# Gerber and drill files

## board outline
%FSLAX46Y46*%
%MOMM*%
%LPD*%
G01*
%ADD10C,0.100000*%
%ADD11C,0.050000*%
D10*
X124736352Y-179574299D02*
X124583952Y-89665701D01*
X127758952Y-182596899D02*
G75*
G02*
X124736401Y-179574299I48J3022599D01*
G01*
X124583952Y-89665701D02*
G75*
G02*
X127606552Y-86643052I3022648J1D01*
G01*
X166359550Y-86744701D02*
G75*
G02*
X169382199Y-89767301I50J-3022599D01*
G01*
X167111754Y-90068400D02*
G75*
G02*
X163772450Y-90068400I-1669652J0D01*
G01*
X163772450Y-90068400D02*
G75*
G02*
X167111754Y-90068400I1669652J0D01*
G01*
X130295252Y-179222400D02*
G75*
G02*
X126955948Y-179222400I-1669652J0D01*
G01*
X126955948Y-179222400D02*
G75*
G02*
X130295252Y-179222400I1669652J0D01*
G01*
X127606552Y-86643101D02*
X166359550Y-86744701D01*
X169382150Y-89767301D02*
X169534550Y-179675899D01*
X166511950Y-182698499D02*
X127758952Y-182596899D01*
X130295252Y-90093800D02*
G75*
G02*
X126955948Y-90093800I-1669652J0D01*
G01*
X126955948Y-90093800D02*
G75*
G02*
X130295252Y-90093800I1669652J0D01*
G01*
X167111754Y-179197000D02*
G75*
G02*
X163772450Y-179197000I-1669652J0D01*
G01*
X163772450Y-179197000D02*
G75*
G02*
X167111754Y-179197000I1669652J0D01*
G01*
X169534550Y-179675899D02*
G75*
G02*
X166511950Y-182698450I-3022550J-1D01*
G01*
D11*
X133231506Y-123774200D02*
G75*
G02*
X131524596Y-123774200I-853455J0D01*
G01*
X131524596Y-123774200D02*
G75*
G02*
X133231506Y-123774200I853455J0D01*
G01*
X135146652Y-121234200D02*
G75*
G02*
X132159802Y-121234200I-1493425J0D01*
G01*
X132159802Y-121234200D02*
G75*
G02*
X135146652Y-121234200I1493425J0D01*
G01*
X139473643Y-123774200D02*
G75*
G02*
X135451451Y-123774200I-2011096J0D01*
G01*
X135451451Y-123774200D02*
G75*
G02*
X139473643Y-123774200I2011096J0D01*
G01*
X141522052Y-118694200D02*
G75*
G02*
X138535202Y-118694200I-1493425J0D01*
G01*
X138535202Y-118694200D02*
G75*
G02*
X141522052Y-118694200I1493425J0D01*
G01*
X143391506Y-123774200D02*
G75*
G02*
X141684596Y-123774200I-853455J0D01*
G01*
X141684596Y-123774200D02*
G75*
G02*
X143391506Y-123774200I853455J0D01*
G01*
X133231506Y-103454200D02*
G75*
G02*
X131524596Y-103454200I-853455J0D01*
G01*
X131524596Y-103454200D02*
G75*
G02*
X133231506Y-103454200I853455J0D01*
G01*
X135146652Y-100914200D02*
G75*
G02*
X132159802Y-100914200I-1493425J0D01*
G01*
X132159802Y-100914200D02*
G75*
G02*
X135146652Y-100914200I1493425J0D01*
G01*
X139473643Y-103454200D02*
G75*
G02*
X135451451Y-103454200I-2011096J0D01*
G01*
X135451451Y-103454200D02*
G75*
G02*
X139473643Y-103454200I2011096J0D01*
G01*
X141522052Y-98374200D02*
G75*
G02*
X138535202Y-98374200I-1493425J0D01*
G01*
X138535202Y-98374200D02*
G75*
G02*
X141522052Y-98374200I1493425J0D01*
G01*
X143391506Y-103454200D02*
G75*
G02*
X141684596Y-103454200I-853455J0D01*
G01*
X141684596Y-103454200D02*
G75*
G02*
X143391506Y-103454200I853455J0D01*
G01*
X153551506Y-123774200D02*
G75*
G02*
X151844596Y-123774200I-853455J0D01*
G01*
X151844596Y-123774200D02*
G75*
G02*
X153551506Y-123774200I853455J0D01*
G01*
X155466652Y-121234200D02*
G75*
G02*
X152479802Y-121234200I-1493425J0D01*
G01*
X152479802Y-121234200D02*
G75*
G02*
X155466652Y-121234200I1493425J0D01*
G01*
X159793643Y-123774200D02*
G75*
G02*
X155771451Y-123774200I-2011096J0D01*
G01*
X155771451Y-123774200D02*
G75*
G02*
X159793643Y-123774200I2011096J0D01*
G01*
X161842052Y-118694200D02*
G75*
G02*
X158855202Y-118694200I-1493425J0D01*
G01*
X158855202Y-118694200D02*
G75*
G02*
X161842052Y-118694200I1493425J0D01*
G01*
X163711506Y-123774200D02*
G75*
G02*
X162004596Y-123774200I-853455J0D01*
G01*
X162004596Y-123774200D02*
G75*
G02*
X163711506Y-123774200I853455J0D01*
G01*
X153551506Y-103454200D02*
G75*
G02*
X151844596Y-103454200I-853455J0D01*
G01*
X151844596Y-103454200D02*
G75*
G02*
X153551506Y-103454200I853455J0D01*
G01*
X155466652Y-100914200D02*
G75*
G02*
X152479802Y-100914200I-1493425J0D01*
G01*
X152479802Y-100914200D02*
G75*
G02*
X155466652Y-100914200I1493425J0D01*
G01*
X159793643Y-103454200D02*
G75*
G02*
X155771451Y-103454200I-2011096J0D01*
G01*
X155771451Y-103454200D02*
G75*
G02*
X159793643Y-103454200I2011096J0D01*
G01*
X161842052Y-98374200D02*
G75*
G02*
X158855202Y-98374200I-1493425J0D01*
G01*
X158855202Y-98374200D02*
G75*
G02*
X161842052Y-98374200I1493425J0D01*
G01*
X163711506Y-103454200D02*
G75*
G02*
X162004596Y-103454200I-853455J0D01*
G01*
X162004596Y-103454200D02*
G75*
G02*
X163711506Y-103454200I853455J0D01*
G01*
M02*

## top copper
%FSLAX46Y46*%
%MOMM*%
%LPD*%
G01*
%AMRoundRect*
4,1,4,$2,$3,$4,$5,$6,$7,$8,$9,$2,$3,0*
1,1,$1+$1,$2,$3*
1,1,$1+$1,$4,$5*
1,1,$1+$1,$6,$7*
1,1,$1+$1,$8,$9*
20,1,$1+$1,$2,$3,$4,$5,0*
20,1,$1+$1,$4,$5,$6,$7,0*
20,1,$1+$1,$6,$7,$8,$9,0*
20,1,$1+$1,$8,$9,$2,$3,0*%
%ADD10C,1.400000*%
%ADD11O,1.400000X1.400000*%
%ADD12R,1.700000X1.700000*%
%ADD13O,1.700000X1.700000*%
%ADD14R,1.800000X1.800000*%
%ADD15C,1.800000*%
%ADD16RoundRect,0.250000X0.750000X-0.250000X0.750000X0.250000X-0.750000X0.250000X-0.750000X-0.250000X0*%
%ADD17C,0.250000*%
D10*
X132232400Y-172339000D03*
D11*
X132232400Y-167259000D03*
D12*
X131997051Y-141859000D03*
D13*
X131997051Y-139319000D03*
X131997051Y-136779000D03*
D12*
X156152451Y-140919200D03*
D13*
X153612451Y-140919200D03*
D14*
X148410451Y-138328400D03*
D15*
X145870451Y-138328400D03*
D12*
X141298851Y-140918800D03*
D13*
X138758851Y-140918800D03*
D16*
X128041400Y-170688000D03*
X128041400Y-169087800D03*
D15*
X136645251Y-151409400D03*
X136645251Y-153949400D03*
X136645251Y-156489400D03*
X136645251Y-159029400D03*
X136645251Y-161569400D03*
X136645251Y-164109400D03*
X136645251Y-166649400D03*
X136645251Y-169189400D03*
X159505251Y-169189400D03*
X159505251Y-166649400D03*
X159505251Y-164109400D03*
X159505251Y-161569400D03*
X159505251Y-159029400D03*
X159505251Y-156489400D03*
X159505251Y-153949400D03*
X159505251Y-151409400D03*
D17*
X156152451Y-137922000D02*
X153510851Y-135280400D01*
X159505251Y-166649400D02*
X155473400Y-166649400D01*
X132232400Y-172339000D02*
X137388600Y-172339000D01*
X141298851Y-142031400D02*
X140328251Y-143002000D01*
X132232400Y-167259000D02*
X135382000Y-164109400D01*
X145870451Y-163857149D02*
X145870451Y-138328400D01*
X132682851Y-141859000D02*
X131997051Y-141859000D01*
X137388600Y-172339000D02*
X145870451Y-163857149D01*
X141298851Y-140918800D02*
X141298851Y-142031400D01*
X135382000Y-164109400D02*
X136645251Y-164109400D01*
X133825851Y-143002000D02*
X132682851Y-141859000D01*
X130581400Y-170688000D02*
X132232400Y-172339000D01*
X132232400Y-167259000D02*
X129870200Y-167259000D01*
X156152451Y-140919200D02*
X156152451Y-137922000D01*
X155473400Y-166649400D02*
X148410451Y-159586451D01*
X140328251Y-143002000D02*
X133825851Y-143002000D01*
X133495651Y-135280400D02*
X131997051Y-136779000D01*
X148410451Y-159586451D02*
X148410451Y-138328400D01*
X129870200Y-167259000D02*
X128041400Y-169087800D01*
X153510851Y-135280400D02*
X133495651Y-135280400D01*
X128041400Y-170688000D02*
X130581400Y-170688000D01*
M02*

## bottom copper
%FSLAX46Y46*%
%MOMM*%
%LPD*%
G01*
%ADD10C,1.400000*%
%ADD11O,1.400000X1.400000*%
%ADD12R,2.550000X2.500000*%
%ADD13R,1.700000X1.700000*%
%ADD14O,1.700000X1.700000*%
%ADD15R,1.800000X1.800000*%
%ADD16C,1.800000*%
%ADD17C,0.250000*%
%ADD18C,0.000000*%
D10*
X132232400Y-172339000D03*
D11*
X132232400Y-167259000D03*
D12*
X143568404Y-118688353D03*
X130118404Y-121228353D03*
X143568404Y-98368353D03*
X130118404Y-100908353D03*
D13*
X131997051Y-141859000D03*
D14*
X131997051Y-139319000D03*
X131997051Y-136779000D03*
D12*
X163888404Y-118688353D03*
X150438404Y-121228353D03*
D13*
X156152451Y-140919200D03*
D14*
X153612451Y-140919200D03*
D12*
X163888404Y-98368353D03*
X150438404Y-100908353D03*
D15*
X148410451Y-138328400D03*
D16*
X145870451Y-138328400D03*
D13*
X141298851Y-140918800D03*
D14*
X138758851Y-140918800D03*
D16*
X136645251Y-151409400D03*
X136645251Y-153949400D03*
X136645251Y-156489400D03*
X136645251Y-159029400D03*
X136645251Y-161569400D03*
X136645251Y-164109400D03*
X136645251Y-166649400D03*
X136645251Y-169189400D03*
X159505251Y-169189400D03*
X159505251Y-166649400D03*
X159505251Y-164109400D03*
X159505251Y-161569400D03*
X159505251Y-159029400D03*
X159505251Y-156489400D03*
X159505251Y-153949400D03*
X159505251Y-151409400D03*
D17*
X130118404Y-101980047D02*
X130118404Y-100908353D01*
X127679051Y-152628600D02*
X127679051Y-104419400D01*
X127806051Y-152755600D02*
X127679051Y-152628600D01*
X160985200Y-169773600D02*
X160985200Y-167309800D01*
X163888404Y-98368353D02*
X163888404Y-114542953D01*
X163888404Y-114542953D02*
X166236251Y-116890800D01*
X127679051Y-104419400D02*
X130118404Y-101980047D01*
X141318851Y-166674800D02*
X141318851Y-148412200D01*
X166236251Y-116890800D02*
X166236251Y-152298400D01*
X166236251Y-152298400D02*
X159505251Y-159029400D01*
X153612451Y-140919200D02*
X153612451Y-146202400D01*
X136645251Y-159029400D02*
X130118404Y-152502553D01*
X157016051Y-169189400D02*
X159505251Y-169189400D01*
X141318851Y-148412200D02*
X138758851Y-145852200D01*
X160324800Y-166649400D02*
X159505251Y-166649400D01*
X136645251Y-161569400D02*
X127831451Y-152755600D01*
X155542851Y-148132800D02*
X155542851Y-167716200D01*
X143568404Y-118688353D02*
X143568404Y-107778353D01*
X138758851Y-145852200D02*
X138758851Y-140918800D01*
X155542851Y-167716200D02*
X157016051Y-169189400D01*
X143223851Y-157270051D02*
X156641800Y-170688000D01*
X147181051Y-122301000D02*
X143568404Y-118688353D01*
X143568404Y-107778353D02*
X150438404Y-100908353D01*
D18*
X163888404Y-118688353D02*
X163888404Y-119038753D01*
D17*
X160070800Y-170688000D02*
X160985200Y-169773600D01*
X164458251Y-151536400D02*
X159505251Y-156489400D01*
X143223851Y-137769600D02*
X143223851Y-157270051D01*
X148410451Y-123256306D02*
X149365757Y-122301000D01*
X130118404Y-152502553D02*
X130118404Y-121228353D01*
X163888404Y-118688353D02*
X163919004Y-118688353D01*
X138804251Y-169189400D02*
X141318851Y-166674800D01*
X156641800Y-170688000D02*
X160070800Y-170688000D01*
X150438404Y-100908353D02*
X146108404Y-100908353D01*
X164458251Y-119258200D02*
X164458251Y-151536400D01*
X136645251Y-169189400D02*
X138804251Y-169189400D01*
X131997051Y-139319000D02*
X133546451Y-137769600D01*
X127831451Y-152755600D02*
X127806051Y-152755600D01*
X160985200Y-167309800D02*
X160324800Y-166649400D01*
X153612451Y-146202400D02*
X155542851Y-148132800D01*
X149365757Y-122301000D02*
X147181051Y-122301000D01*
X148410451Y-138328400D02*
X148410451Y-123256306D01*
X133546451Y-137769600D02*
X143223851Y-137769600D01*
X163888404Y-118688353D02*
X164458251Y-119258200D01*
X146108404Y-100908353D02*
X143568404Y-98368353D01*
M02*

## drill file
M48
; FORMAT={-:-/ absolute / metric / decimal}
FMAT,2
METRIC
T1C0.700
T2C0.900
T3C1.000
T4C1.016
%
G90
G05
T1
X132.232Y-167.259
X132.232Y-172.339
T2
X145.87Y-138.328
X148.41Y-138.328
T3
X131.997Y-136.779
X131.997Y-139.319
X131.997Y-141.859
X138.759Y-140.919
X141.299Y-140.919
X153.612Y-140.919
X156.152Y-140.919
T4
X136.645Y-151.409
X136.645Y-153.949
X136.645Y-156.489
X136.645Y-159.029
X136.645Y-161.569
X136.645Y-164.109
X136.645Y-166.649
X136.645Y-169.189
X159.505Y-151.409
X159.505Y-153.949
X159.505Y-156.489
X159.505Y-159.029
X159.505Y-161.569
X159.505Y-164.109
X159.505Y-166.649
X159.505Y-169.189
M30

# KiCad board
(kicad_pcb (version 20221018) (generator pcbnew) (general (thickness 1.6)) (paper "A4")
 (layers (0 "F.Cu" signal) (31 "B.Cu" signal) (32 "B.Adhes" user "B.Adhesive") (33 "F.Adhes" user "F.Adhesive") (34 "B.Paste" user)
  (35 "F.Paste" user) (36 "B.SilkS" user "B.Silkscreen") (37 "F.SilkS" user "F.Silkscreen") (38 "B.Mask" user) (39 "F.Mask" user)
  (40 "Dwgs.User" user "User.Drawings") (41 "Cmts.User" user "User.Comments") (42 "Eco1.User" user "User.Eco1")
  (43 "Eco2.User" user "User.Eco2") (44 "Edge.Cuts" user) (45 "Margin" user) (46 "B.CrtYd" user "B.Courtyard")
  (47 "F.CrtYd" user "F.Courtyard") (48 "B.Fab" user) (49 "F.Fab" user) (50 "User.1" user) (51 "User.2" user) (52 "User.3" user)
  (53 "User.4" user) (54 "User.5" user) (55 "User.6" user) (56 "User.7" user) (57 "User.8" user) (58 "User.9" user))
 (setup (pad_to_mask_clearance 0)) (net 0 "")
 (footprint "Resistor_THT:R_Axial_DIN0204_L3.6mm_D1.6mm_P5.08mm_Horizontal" (layer "F.Cu") (at 132.2324 172.339 90)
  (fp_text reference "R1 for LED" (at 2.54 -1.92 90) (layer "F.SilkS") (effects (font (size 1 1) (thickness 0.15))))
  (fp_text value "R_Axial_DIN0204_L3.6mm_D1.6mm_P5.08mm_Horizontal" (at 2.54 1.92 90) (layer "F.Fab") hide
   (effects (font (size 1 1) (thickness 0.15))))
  (pad "1" thru_hole circle (at 0 0 90) (size 1.4 1.4) (drill 0.7) (layers "*.Cu" "*.Mask"))
  (pad "2" thru_hole oval (at 5.08 0 90) (size 1.4 1.4) (drill 0.7) (layers "*.Cu" "*.Mask")))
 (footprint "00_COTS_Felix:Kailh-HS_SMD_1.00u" (layer "F.Cu") (at 137.458051 123.7742)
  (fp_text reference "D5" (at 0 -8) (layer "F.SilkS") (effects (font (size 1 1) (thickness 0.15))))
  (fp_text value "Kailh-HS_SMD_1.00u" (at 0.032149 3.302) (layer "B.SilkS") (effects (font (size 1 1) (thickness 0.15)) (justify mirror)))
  (fp_circle (center -5.08 0) (end -4.572 -0.6858) (stroke (width 0.05) (type default)) (fill none) (layer "Edge.Cuts"))
  (fp_circle (center -3.804824 -2.54) (end -2.687224 -3.5306) (stroke (width 0.05) (type default)) (fill none) (layer "Edge.Cuts"))
  (fp_circle (center 0.004496 0) (end 0.944296 -1.778) (stroke (width 0.05) (type default)) (fill none) (layer "Edge.Cuts"))
  (fp_circle (center 2.570576 -5.08) (end 4.064001 -5.08) (stroke (width 0.05) (type default)) (fill none) (layer "Edge.Cuts"))
  (fp_circle (center 5.08 0) (end 5.588 -0.6858) (stroke (width 0.05) (type default)) (fill none) (layer "Edge.Cuts"))
  (pad "1" smd rect (at 6.110353 -5.085847) (size 2.55 2.5) (layers "B.Cu" "F.Paste" "F.Mask") (solder_mask_margin 0.102))
  (pad "2" smd rect (at -7.339647 -2.545847) (size 2.55 2.5) (layers "B.Cu" "F.Paste" "F.Mask") (solder_mask_margin 0.102)))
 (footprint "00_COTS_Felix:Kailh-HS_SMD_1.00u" (layer "F.Cu") (at 137.458051 103.4542)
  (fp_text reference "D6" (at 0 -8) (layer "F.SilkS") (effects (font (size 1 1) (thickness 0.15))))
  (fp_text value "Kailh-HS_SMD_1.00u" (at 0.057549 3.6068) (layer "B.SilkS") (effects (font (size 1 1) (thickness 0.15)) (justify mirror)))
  (fp_circle (center -5.08 0) (end -4.572 -0.6858) (stroke (width 0.05) (type default)) (fill none) (layer "Edge.Cuts"))
  (fp_circle (center -3.804824 -2.54) (end -2.687224 -3.5306) (stroke (width 0.05) (type default)) (fill none) (layer "Edge.Cuts"))
  (fp_circle (center 0.004496 0) (end 0.944296 -1.778) (stroke (width 0.05) (type default)) (fill none) (layer "Edge.Cuts"))
  (fp_circle (center 2.570576 -5.08) (end 4.064001 -5.08) (stroke (width 0.05) (type default)) (fill none) (layer "Edge.Cuts"))
  (fp_circle (center 5.08 0) (end 5.588 -0.6858) (stroke (width 0.05) (type default)) (fill none) (layer "Edge.Cuts"))
  (pad "1" smd rect (at 6.110353 -5.085847) (size 2.55 2.5) (layers "B.Cu" "F.Paste" "F.Mask") (solder_mask_margin 0.102))
  (pad "2" smd rect (at -7.339647 -2.545847) (size 2.55 2.5) (layers "B.Cu" "F.Paste" "F.Mask") (solder_mask_margin 0.102)))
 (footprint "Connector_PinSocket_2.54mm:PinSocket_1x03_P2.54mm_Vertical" (layer "F.Cu") (at 131.997051 141.859 180)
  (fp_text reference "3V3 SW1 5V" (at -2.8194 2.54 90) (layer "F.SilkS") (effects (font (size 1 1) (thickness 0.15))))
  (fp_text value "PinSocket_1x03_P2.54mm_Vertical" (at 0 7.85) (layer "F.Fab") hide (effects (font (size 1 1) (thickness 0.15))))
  (pad "1" thru_hole rect (at 0 0 180) (size 1.7 1.7) (drill 1) (layers "*.Cu" "*.Mask"))
  (pad "2" thru_hole oval (at 0 2.54 180) (size 1.7 1.7) (drill 1) (layers "*.Cu" "*.Mask"))
  (pad "3" thru_hole oval (at 0 5.08 180) (size 1.7 1.7) (drill 1) (layers "*.Cu" "*.Mask")))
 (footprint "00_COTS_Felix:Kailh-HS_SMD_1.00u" (layer "F.Cu") (at 157.778051 123.7742)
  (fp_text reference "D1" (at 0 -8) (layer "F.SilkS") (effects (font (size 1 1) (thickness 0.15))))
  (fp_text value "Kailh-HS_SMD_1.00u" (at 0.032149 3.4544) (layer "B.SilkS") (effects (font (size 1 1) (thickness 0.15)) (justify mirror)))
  (fp_circle (center -5.08 0) (end -4.572 -0.6858) (stroke (width 0.05) (type default)) (fill none) (layer "Edge.Cuts"))
  (fp_circle (center -3.804824 -2.54) (end -2.687224 -3.5306) (stroke (width 0.05) (type default)) (fill none) (layer "Edge.Cuts"))
  (fp_circle (center 0.004496 0) (end 0.944296 -1.778) (stroke (width 0.05) (type default)) (fill none) (layer "Edge.Cuts"))
  (fp_circle (center 2.570576 -5.08) (end 4.064001 -5.08) (stroke (width 0.05) (type default)) (fill none) (layer "Edge.Cuts"))
  (fp_circle (center 5.08 0) (end 5.588 -0.6858) (stroke (width 0.05) (type default)) (fill none) (layer "Edge.Cuts"))
  (pad "1" smd rect (at 6.110353 -5.085847) (size 2.55 2.5) (layers "B.Cu" "F.Paste" "F.Mask") (solder_mask_margin 0.102))
  (pad "2" smd rect (at -7.339647 -2.545847) (size 2.55 2.5) (layers "B.Cu" "F.Paste" "F.Mask") (solder_mask_margin 0.102)))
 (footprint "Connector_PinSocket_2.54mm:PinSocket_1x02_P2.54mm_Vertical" (layer "F.Cu") (at 156.152451 140.9192 -90)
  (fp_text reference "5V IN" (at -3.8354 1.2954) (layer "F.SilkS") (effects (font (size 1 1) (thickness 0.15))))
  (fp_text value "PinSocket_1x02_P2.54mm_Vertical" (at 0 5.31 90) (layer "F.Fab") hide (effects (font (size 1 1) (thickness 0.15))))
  (pad "1" thru_hole rect (at 0 0 270) (size 1.7 1.7) (drill 1) (layers "*.Cu" "*.Mask"))
  (pad "2" thru_hole oval (at 0 2.54 270) (size 1.7 1.7) (drill 1) (layers "*.Cu" "*.Mask")))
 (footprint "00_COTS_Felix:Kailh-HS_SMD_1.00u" (layer "F.Cu") (at 157.778051 103.4542)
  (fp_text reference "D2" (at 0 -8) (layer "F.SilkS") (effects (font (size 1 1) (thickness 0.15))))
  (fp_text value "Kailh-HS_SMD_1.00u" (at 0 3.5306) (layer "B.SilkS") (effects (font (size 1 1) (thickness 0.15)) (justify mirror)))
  (fp_circle (center -5.08 0) (end -4.572 -0.6858) (stroke (width 0.05) (type default)) (fill none) (layer "Edge.Cuts"))
  (fp_circle (center -3.804824 -2.54) (end -2.687224 -3.5306) (stroke (width 0.05) (type default)) (fill none) (layer "Edge.Cuts"))
  (fp_circle (center 0.004496 0) (end 0.944296 -1.778) (stroke (width 0.05) (type default)) (fill none) (layer "Edge.Cuts"))
  (fp_circle (center 2.570576 -5.08) (end 4.064001 -5.08) (stroke (width 0.05) (type default)) (fill none) (layer "Edge.Cuts"))
  (fp_circle (center 5.08 0) (end 5.588 -0.6858) (stroke (width 0.05) (type default)) (fill none) (layer "Edge.Cuts"))
  (pad "1" smd rect (at 6.110353 -5.085847) (size 2.55 2.5) (layers "B.Cu" "F.Paste" "F.Mask") (solder_mask_margin 0.102))
  (pad "2" smd rect (at -7.339647 -2.545847) (size 2.55 2.5) (layers "B.Cu" "F.Paste" "F.Mask") (solder_mask_margin 0.102)))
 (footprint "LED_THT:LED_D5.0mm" (layer "F.Cu") (at 148.410451 138.3284 180)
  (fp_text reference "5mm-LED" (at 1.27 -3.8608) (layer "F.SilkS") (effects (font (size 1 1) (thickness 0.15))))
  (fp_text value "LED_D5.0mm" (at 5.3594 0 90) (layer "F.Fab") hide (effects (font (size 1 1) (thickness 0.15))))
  (pad "1" thru_hole rect (at 0 0 180) (size 1.8 1.8) (drill 0.9) (layers "*.Cu" "*.Mask"))
  (pad "2" thru_hole circle (at 2.54 0 180) (size 1.8 1.8) (drill 0.9) (layers "*.Cu" "*.Mask")))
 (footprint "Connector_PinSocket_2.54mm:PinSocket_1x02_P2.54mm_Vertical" (layer "F.Cu") (at 141.298851 140.9188 -90)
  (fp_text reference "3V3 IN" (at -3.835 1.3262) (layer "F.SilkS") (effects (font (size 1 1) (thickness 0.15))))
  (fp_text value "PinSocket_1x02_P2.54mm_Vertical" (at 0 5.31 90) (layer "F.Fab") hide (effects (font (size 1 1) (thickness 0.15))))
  (pad "1" thru_hole rect (at 0 0 270) (size 1.7 1.7) (drill 1) (layers "*.Cu" "*.Mask"))
  (pad "2" thru_hole oval (at 0 2.54 270) (size 1.7 1.7) (drill 1) (layers "*.Cu" "*.Mask")))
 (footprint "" (layer "F.Cu") (at 128.0414 170.688)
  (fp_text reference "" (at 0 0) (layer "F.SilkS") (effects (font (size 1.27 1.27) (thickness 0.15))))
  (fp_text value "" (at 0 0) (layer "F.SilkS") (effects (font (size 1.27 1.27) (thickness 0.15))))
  (pad "1" smd roundrect (at 0 0 90) (size 1 2) (layers "F.Cu" "F.Paste" "F.Mask") (roundrect_rratio 0.25)))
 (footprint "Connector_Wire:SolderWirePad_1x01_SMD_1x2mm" (layer "F.Cu") (at 128.0414 169.0878 90)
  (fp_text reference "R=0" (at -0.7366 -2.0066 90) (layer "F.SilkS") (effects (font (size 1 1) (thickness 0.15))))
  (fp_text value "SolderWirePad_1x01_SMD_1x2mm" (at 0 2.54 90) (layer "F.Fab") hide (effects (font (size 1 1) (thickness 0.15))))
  (pad "1" smd roundrect (at 0 0 90) (size 1 2) (layers "F.Cu" "F.Paste" "F.Mask") (roundrect_rratio 0.25)))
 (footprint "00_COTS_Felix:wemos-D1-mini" (layer "F.Cu") (at 148.088051 160.6542)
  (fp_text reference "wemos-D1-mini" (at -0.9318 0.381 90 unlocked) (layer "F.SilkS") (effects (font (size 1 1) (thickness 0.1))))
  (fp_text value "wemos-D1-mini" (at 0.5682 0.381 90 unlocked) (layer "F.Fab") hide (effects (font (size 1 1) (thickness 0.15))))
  (pad "1" thru_hole circle (at -11.4428 -9.2448 90) (size 1.8 1.8) (drill 1.016) (layers "*.Cu" "*.Mask"))
  (pad "2" thru_hole circle (at -11.4428 -6.7048 90) (size 1.8 1.8) (drill 1.016) (layers "*.Cu" "*.Mask"))
  (pad "3" thru_hole circle (at -11.4428 -4.1648 90) (size 1.8 1.8) (drill 1.016) (layers "*.Cu" "*.Mask"))
  (pad "4" thru_hole circle (at -11.4428 -1.6248 90) (size 1.8 1.8) (drill 1.016) (layers "*.Cu" "*.Mask"))
  (pad "5" thru_hole circle (at -11.4428 0.9152 90) (size 1.8 1.8) (drill 1.016) (layers "*.Cu" "*.Mask"))
  (pad "6" thru_hole circle (at -11.4428 3.4552 90) (size 1.8 1.8) (drill 1.016) (layers "*.Cu" "*.Mask"))
  (pad "7" thru_hole circle (at -11.4428 5.9952 90) (size 1.8 1.8) (drill 1.016) (layers "*.Cu" "*.Mask"))
  (pad "8" thru_hole circle (at -11.4428 8.5352 90) (size 1.8 1.8) (drill 1.016) (layers "*.Cu" "*.Mask"))
  (pad "9" thru_hole circle (at 11.4172 8.5352 90) (size 1.8 1.8) (drill 1.016) (layers "*.Cu" "*.Mask"))
  (pad "10" thru_hole circle (at 11.4172 5.9952 90) (size 1.8 1.8) (drill 1.016) (layers "*.Cu" "*.Mask"))
  (pad "11" thru_hole circle (at 11.4172 3.4552 90) (size 1.8 1.8) (drill 1.016) (layers "*.Cu" "*.Mask"))
  (pad "12" thru_hole circle (at 11.4172 0.9152 90) (size 1.8 1.8) (drill 1.016) (layers "*.Cu" "*.Mask"))
  (pad "13" thru_hole circle (at 11.4172 -1.6248 90) (size 1.8 1.8) (drill 1.016) (layers "*.Cu" "*.Mask"))
  (pad "14" thru_hole circle (at 11.4172 -4.1648 90) (size 1.8 1.8) (drill 1.016) (layers "*.Cu" "*.Mask"))
  (pad "15" thru_hole circle (at 11.4172 -6.7048 90) (size 1.8 1.8) (drill 1.016) (layers "*.Cu" "*.Mask"))
  (pad "16" thru_hole circle (at 11.4172 -9.2448 90) (size 1.8 1.8) (drill 1.016) (layers "*.Cu" "*.Mask")))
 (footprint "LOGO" (layer "B.Cu") (at 147.2184 114.0206 180)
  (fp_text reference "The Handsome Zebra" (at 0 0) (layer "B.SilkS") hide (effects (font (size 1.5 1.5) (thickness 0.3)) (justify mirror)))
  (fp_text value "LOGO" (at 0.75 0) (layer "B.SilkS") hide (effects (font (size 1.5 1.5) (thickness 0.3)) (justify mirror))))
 (gr_line (start 124.736352 179.574299) (end 124.583952 89.665701) (stroke (width 0.1) (type default)) (layer "Edge.Cuts"))
 (gr_arc (start 127.758952 182.596899) (mid 125.621651 181.7116) (end 124.736352 179.574299) (stroke (width 0.1) (type default))
  (layer "Edge.Cuts"))
 (gr_arc (start 124.583952 89.665701) (mid 125.469251 87.5284) (end 127.606552 86.643101) (stroke (width 0.1) (type default))
  (layer "Edge.Cuts"))
 (gr_arc (start 166.35955 86.744701) (mid 168.496851 87.63) (end 169.38215 89.767301) (stroke (width 0.1) (type default))
  (layer "Edge.Cuts"))
 (gr_circle (center 165.442102 90.0684) (end 166.839102 89.154) (stroke (width 0.1) (type default)) (fill none) (layer "Edge.Cuts"))
 (gr_circle (center 128.6256 179.2224) (end 130.0226 178.308) (stroke (width 0.1) (type default)) (fill none) (layer "Edge.Cuts"))
 (gr_line (start 127.606552 86.643101) (end 166.35955 86.744701) (stroke (width 0.1) (type default)) (layer "Edge.Cuts"))
 (gr_line (start 169.38215 89.767301) (end 169.53455 179.675899) (stroke (width 0.1) (type default)) (layer "Edge.Cuts"))
 (gr_line (start 166.51195 182.698499) (end 127.758952 182.596899) (stroke (width 0.1) (type default)) (layer "Edge.Cuts"))
 (gr_circle (center 128.6256 90.0938) (end 130.0226 89.1794) (stroke (width 0.1) (type default)) (fill none) (layer "Edge.Cuts"))
 (gr_circle (center 165.442102 179.197) (end 166.839102 178.2826) (stroke (width 0.1) (type default)) (fill none) (layer "Edge.Cuts"))
 (gr_arc (start 169.53455 179.675899) (mid 168.649251 181.8132) (end 166.51195 182.698499) (stroke (width 0.1) (type default))
  (layer "Edge.Cuts"))
 (segment (start 156.152451 137.922) (end 153.510851 135.2804) (width 0.25) (layer "F.Cu") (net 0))
 (segment (start 159.505251 166.6494) (end 155.4734 166.6494) (width 0.25) (layer "F.Cu") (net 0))
 (segment (start 132.2324 172.339) (end 137.3886 172.339) (width 0.25) (layer "F.Cu") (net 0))
 (segment (start 141.298851 142.0314) (end 140.328251 143.002) (width 0.25) (layer "F.Cu") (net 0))
 (segment (start 132.2324 167.259) (end 135.382 164.1094) (width 0.25) (layer "F.Cu") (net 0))
 (segment (start 145.870451 163.857149) (end 145.870451 138.3284) (width 0.25) (layer "F.Cu") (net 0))
 (segment (start 132.682851 141.859) (end 131.997051 141.859) (width 0.25) (layer "F.Cu") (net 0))
 (segment (start 137.3886 172.339) (end 145.870451 163.857149) (width 0.25) (layer "F.Cu") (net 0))
 (segment (start 141.298851 140.9188) (end 141.298851 142.0314) (width 0.25) (layer "F.Cu") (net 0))
 (segment (start 135.382 164.1094) (end 136.645251 164.1094) (width 0.25) (layer "F.Cu") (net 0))
 (segment (start 133.825851 143.002) (end 132.682851 141.859) (width 0.25) (layer "F.Cu") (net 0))
 (segment (start 130.5814 170.688) (end 132.2324 172.339) (width 0.25) (layer "F.Cu") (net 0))
 (segment (start 132.2324 167.259) (end 129.8702 167.259) (width 0.25) (layer "F.Cu") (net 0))
 (segment (start 156.152451 140.9192) (end 156.152451 137.922) (width 0.25) (layer "F.Cu") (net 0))
 (segment (start 155.4734 166.6494) (end 148.410451 159.586451) (width 0.25) (layer "F.Cu") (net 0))
 (segment (start 140.328251 143.002) (end 133.825851 143.002) (width 0.25) (layer "F.Cu") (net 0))
 (segment (start 133.495651 135.2804) (end 131.997051 136.779) (width 0.25) (layer "F.Cu") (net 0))
 (segment (start 148.410451 159.586451) (end 148.410451 138.3284) (width 0.25) (layer "F.Cu") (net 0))
 (segment (start 129.8702 167.259) (end 128.0414 169.0878) (width 0.25) (layer "F.Cu") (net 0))
 (segment (start 153.510851 135.2804) (end 133.495651 135.2804) (width 0.25) (layer "F.Cu") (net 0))
 (segment (start 128.0414 170.688) (end 130.5814 170.688) (width 0.25) (layer "F.Cu") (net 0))
 (segment (start 130.118404 101.980047) (end 130.118404 100.908353) (width 0.25) (layer "B.Cu") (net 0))
 (segment (start 127.679051 152.6286) (end 127.679051 104.4194) (width 0.25) (layer "B.Cu") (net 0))
 (segment (start 127.806051 152.7556) (end 127.679051 152.6286) (width 0.25) (layer "B.Cu") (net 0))
 (segment (start 160.9852 169.7736) (end 160.9852 167.3098) (width 0.25) (layer "B.Cu") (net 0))
 (segment (start 163.888404 98.368353) (end 163.888404 114.542953) (width 0.25) (layer "B.Cu") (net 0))
 (segment (start 163.888404 114.542953) (end 166.236251 116.8908) (width 0.25) (layer "B.Cu") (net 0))
 (segment (start 127.679051 104.4194) (end 130.118404 101.980047) (width 0.25) (layer "B.Cu") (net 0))
 (segment (start 141.318851 166.6748) (end 141.318851 148.4122) (width 0.25) (layer "B.Cu") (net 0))
 (segment (start 166.236251 116.8908) (end 166.236251 152.2984) (width 0.25) (layer "B.Cu") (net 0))
 (segment (start 166.236251 152.2984) (end 159.505251 159.0294) (width 0.25) (layer "B.Cu") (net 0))
 (segment (start 153.612451 140.9192) (end 153.612451 146.2024) (width 0.25) (layer "B.Cu") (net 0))
 (segment (start 136.645251 159.0294) (end 130.118404 152.502553) (width 0.25) (layer "B.Cu") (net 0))
 (segment (start 157.016051 169.1894) (end 159.505251 169.1894) (width 0.25) (layer "B.Cu") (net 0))
 (segment (start 141.318851 148.4122) (end 138.758851 145.8522) (width 0.25) (layer "B.Cu") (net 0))
 (segment (start 160.3248 166.6494) (end 159.505251 166.6494) (width 0.25) (layer "B.Cu") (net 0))
 (segment (start 136.645251 161.5694) (end 127.831451 152.7556) (width 0.25) (layer "B.Cu") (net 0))
 (segment (start 155.542851 148.1328) (end 155.542851 167.7162) (width 0.25) (layer "B.Cu") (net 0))
 (segment (start 143.568404 118.688353) (end 143.568404 107.778353) (width 0.25) (layer "B.Cu") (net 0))
 (segment (start 138.758851 145.8522) (end 138.758851 140.9188) (width 0.25) (layer "B.Cu") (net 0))
 (segment (start 155.542851 167.7162) (end 157.016051 169.1894) (width 0.25) (layer "B.Cu") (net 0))
 (segment (start 143.223851 157.270051) (end 156.6418 170.688) (width 0.25) (layer "B.Cu") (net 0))
 (segment (start 147.181051 122.301) (end 143.568404 118.688353) (width 0.25) (layer "B.Cu") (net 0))
 (segment (start 143.568404 107.778353) (end 150.438404 100.908353) (width 0.25) (layer "B.Cu") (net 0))
 (segment (start 163.888404 118.688353) (end 163.888404 119.038753) (width 0) (layer "B.Cu") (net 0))
 (segment (start 160.0708 170.688) (end 160.9852 169.7736) (width 0.25) (layer "B.Cu") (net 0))
 (segment (start 164.458251 151.5364) (end 159.505251 156.4894) (width 0.25) (layer "B.Cu") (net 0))
 (segment (start 143.223851 137.7696) (end 143.223851 157.270051) (width 0.25) (layer "B.Cu") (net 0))
 (segment (start 148.410451 123.256306) (end 149.365757 122.301) (width 0.25) (layer "B.Cu") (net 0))
 (segment (start 130.118404 152.502553) (end 130.118404 121.228353) (width 0.25) (layer "B.Cu") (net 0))
 (segment (start 163.888404 118.688353) (end 163.919004 118.688353) (width 0.25) (layer "B.Cu") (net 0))
 (segment (start 138.804251 169.1894) (end 141.318851 166.6748) (width 0.25) (layer "B.Cu") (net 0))
 (segment (start 156.6418 170.688) (end 160.0708 170.688) (width 0.25) (layer "B.Cu") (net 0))
 (segment (start 150.438404 100.908353) (end 146.108404 100.908353) (width 0.25) (layer "B.Cu") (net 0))
 (segment (start 164.458251 119.2582) (end 164.458251 151.5364) (width 0.25) (layer "B.Cu") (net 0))
 (segment (start 136.645251 169.1894) (end 138.804251 169.1894) (width 0.25) (layer "B.Cu") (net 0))
 (segment (start 131.997051 139.319) (end 133.546451 137.7696) (width 0.25) (layer "B.Cu") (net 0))
 (segment (start 127.831451 152.7556) (end 127.806051 152.7556) (width 0.25) (layer "B.Cu") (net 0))
 (segment (start 160.9852 167.3098) (end 160.3248 166.6494) (width 0.25) (layer "B.Cu") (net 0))
 (segment (start 153.612451 146.2024) (end 155.542851 148.1328) (width 0.25) (layer "B.Cu") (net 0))
 (segment (start 149.365757 122.301) (end 147.181051 122.301) (width 0.25) (layer "B.Cu") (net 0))
 (segment (start 148.410451 138.3284) (end 148.410451 123.256306) (width 0.25) (layer "B.Cu") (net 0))
 (segment (start 133.546451 137.7696) (end 143.223851 137.7696) (width 0.25) (layer "B.Cu") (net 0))
 (segment (start 163.888404 118.688353) (end 164.458251 119.2582) (width 0.25) (layer "B.Cu") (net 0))
 (segment (start 146.108404 100.908353) (end 143.568404 98.368353) (width 0.25) (layer "B.Cu") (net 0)))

